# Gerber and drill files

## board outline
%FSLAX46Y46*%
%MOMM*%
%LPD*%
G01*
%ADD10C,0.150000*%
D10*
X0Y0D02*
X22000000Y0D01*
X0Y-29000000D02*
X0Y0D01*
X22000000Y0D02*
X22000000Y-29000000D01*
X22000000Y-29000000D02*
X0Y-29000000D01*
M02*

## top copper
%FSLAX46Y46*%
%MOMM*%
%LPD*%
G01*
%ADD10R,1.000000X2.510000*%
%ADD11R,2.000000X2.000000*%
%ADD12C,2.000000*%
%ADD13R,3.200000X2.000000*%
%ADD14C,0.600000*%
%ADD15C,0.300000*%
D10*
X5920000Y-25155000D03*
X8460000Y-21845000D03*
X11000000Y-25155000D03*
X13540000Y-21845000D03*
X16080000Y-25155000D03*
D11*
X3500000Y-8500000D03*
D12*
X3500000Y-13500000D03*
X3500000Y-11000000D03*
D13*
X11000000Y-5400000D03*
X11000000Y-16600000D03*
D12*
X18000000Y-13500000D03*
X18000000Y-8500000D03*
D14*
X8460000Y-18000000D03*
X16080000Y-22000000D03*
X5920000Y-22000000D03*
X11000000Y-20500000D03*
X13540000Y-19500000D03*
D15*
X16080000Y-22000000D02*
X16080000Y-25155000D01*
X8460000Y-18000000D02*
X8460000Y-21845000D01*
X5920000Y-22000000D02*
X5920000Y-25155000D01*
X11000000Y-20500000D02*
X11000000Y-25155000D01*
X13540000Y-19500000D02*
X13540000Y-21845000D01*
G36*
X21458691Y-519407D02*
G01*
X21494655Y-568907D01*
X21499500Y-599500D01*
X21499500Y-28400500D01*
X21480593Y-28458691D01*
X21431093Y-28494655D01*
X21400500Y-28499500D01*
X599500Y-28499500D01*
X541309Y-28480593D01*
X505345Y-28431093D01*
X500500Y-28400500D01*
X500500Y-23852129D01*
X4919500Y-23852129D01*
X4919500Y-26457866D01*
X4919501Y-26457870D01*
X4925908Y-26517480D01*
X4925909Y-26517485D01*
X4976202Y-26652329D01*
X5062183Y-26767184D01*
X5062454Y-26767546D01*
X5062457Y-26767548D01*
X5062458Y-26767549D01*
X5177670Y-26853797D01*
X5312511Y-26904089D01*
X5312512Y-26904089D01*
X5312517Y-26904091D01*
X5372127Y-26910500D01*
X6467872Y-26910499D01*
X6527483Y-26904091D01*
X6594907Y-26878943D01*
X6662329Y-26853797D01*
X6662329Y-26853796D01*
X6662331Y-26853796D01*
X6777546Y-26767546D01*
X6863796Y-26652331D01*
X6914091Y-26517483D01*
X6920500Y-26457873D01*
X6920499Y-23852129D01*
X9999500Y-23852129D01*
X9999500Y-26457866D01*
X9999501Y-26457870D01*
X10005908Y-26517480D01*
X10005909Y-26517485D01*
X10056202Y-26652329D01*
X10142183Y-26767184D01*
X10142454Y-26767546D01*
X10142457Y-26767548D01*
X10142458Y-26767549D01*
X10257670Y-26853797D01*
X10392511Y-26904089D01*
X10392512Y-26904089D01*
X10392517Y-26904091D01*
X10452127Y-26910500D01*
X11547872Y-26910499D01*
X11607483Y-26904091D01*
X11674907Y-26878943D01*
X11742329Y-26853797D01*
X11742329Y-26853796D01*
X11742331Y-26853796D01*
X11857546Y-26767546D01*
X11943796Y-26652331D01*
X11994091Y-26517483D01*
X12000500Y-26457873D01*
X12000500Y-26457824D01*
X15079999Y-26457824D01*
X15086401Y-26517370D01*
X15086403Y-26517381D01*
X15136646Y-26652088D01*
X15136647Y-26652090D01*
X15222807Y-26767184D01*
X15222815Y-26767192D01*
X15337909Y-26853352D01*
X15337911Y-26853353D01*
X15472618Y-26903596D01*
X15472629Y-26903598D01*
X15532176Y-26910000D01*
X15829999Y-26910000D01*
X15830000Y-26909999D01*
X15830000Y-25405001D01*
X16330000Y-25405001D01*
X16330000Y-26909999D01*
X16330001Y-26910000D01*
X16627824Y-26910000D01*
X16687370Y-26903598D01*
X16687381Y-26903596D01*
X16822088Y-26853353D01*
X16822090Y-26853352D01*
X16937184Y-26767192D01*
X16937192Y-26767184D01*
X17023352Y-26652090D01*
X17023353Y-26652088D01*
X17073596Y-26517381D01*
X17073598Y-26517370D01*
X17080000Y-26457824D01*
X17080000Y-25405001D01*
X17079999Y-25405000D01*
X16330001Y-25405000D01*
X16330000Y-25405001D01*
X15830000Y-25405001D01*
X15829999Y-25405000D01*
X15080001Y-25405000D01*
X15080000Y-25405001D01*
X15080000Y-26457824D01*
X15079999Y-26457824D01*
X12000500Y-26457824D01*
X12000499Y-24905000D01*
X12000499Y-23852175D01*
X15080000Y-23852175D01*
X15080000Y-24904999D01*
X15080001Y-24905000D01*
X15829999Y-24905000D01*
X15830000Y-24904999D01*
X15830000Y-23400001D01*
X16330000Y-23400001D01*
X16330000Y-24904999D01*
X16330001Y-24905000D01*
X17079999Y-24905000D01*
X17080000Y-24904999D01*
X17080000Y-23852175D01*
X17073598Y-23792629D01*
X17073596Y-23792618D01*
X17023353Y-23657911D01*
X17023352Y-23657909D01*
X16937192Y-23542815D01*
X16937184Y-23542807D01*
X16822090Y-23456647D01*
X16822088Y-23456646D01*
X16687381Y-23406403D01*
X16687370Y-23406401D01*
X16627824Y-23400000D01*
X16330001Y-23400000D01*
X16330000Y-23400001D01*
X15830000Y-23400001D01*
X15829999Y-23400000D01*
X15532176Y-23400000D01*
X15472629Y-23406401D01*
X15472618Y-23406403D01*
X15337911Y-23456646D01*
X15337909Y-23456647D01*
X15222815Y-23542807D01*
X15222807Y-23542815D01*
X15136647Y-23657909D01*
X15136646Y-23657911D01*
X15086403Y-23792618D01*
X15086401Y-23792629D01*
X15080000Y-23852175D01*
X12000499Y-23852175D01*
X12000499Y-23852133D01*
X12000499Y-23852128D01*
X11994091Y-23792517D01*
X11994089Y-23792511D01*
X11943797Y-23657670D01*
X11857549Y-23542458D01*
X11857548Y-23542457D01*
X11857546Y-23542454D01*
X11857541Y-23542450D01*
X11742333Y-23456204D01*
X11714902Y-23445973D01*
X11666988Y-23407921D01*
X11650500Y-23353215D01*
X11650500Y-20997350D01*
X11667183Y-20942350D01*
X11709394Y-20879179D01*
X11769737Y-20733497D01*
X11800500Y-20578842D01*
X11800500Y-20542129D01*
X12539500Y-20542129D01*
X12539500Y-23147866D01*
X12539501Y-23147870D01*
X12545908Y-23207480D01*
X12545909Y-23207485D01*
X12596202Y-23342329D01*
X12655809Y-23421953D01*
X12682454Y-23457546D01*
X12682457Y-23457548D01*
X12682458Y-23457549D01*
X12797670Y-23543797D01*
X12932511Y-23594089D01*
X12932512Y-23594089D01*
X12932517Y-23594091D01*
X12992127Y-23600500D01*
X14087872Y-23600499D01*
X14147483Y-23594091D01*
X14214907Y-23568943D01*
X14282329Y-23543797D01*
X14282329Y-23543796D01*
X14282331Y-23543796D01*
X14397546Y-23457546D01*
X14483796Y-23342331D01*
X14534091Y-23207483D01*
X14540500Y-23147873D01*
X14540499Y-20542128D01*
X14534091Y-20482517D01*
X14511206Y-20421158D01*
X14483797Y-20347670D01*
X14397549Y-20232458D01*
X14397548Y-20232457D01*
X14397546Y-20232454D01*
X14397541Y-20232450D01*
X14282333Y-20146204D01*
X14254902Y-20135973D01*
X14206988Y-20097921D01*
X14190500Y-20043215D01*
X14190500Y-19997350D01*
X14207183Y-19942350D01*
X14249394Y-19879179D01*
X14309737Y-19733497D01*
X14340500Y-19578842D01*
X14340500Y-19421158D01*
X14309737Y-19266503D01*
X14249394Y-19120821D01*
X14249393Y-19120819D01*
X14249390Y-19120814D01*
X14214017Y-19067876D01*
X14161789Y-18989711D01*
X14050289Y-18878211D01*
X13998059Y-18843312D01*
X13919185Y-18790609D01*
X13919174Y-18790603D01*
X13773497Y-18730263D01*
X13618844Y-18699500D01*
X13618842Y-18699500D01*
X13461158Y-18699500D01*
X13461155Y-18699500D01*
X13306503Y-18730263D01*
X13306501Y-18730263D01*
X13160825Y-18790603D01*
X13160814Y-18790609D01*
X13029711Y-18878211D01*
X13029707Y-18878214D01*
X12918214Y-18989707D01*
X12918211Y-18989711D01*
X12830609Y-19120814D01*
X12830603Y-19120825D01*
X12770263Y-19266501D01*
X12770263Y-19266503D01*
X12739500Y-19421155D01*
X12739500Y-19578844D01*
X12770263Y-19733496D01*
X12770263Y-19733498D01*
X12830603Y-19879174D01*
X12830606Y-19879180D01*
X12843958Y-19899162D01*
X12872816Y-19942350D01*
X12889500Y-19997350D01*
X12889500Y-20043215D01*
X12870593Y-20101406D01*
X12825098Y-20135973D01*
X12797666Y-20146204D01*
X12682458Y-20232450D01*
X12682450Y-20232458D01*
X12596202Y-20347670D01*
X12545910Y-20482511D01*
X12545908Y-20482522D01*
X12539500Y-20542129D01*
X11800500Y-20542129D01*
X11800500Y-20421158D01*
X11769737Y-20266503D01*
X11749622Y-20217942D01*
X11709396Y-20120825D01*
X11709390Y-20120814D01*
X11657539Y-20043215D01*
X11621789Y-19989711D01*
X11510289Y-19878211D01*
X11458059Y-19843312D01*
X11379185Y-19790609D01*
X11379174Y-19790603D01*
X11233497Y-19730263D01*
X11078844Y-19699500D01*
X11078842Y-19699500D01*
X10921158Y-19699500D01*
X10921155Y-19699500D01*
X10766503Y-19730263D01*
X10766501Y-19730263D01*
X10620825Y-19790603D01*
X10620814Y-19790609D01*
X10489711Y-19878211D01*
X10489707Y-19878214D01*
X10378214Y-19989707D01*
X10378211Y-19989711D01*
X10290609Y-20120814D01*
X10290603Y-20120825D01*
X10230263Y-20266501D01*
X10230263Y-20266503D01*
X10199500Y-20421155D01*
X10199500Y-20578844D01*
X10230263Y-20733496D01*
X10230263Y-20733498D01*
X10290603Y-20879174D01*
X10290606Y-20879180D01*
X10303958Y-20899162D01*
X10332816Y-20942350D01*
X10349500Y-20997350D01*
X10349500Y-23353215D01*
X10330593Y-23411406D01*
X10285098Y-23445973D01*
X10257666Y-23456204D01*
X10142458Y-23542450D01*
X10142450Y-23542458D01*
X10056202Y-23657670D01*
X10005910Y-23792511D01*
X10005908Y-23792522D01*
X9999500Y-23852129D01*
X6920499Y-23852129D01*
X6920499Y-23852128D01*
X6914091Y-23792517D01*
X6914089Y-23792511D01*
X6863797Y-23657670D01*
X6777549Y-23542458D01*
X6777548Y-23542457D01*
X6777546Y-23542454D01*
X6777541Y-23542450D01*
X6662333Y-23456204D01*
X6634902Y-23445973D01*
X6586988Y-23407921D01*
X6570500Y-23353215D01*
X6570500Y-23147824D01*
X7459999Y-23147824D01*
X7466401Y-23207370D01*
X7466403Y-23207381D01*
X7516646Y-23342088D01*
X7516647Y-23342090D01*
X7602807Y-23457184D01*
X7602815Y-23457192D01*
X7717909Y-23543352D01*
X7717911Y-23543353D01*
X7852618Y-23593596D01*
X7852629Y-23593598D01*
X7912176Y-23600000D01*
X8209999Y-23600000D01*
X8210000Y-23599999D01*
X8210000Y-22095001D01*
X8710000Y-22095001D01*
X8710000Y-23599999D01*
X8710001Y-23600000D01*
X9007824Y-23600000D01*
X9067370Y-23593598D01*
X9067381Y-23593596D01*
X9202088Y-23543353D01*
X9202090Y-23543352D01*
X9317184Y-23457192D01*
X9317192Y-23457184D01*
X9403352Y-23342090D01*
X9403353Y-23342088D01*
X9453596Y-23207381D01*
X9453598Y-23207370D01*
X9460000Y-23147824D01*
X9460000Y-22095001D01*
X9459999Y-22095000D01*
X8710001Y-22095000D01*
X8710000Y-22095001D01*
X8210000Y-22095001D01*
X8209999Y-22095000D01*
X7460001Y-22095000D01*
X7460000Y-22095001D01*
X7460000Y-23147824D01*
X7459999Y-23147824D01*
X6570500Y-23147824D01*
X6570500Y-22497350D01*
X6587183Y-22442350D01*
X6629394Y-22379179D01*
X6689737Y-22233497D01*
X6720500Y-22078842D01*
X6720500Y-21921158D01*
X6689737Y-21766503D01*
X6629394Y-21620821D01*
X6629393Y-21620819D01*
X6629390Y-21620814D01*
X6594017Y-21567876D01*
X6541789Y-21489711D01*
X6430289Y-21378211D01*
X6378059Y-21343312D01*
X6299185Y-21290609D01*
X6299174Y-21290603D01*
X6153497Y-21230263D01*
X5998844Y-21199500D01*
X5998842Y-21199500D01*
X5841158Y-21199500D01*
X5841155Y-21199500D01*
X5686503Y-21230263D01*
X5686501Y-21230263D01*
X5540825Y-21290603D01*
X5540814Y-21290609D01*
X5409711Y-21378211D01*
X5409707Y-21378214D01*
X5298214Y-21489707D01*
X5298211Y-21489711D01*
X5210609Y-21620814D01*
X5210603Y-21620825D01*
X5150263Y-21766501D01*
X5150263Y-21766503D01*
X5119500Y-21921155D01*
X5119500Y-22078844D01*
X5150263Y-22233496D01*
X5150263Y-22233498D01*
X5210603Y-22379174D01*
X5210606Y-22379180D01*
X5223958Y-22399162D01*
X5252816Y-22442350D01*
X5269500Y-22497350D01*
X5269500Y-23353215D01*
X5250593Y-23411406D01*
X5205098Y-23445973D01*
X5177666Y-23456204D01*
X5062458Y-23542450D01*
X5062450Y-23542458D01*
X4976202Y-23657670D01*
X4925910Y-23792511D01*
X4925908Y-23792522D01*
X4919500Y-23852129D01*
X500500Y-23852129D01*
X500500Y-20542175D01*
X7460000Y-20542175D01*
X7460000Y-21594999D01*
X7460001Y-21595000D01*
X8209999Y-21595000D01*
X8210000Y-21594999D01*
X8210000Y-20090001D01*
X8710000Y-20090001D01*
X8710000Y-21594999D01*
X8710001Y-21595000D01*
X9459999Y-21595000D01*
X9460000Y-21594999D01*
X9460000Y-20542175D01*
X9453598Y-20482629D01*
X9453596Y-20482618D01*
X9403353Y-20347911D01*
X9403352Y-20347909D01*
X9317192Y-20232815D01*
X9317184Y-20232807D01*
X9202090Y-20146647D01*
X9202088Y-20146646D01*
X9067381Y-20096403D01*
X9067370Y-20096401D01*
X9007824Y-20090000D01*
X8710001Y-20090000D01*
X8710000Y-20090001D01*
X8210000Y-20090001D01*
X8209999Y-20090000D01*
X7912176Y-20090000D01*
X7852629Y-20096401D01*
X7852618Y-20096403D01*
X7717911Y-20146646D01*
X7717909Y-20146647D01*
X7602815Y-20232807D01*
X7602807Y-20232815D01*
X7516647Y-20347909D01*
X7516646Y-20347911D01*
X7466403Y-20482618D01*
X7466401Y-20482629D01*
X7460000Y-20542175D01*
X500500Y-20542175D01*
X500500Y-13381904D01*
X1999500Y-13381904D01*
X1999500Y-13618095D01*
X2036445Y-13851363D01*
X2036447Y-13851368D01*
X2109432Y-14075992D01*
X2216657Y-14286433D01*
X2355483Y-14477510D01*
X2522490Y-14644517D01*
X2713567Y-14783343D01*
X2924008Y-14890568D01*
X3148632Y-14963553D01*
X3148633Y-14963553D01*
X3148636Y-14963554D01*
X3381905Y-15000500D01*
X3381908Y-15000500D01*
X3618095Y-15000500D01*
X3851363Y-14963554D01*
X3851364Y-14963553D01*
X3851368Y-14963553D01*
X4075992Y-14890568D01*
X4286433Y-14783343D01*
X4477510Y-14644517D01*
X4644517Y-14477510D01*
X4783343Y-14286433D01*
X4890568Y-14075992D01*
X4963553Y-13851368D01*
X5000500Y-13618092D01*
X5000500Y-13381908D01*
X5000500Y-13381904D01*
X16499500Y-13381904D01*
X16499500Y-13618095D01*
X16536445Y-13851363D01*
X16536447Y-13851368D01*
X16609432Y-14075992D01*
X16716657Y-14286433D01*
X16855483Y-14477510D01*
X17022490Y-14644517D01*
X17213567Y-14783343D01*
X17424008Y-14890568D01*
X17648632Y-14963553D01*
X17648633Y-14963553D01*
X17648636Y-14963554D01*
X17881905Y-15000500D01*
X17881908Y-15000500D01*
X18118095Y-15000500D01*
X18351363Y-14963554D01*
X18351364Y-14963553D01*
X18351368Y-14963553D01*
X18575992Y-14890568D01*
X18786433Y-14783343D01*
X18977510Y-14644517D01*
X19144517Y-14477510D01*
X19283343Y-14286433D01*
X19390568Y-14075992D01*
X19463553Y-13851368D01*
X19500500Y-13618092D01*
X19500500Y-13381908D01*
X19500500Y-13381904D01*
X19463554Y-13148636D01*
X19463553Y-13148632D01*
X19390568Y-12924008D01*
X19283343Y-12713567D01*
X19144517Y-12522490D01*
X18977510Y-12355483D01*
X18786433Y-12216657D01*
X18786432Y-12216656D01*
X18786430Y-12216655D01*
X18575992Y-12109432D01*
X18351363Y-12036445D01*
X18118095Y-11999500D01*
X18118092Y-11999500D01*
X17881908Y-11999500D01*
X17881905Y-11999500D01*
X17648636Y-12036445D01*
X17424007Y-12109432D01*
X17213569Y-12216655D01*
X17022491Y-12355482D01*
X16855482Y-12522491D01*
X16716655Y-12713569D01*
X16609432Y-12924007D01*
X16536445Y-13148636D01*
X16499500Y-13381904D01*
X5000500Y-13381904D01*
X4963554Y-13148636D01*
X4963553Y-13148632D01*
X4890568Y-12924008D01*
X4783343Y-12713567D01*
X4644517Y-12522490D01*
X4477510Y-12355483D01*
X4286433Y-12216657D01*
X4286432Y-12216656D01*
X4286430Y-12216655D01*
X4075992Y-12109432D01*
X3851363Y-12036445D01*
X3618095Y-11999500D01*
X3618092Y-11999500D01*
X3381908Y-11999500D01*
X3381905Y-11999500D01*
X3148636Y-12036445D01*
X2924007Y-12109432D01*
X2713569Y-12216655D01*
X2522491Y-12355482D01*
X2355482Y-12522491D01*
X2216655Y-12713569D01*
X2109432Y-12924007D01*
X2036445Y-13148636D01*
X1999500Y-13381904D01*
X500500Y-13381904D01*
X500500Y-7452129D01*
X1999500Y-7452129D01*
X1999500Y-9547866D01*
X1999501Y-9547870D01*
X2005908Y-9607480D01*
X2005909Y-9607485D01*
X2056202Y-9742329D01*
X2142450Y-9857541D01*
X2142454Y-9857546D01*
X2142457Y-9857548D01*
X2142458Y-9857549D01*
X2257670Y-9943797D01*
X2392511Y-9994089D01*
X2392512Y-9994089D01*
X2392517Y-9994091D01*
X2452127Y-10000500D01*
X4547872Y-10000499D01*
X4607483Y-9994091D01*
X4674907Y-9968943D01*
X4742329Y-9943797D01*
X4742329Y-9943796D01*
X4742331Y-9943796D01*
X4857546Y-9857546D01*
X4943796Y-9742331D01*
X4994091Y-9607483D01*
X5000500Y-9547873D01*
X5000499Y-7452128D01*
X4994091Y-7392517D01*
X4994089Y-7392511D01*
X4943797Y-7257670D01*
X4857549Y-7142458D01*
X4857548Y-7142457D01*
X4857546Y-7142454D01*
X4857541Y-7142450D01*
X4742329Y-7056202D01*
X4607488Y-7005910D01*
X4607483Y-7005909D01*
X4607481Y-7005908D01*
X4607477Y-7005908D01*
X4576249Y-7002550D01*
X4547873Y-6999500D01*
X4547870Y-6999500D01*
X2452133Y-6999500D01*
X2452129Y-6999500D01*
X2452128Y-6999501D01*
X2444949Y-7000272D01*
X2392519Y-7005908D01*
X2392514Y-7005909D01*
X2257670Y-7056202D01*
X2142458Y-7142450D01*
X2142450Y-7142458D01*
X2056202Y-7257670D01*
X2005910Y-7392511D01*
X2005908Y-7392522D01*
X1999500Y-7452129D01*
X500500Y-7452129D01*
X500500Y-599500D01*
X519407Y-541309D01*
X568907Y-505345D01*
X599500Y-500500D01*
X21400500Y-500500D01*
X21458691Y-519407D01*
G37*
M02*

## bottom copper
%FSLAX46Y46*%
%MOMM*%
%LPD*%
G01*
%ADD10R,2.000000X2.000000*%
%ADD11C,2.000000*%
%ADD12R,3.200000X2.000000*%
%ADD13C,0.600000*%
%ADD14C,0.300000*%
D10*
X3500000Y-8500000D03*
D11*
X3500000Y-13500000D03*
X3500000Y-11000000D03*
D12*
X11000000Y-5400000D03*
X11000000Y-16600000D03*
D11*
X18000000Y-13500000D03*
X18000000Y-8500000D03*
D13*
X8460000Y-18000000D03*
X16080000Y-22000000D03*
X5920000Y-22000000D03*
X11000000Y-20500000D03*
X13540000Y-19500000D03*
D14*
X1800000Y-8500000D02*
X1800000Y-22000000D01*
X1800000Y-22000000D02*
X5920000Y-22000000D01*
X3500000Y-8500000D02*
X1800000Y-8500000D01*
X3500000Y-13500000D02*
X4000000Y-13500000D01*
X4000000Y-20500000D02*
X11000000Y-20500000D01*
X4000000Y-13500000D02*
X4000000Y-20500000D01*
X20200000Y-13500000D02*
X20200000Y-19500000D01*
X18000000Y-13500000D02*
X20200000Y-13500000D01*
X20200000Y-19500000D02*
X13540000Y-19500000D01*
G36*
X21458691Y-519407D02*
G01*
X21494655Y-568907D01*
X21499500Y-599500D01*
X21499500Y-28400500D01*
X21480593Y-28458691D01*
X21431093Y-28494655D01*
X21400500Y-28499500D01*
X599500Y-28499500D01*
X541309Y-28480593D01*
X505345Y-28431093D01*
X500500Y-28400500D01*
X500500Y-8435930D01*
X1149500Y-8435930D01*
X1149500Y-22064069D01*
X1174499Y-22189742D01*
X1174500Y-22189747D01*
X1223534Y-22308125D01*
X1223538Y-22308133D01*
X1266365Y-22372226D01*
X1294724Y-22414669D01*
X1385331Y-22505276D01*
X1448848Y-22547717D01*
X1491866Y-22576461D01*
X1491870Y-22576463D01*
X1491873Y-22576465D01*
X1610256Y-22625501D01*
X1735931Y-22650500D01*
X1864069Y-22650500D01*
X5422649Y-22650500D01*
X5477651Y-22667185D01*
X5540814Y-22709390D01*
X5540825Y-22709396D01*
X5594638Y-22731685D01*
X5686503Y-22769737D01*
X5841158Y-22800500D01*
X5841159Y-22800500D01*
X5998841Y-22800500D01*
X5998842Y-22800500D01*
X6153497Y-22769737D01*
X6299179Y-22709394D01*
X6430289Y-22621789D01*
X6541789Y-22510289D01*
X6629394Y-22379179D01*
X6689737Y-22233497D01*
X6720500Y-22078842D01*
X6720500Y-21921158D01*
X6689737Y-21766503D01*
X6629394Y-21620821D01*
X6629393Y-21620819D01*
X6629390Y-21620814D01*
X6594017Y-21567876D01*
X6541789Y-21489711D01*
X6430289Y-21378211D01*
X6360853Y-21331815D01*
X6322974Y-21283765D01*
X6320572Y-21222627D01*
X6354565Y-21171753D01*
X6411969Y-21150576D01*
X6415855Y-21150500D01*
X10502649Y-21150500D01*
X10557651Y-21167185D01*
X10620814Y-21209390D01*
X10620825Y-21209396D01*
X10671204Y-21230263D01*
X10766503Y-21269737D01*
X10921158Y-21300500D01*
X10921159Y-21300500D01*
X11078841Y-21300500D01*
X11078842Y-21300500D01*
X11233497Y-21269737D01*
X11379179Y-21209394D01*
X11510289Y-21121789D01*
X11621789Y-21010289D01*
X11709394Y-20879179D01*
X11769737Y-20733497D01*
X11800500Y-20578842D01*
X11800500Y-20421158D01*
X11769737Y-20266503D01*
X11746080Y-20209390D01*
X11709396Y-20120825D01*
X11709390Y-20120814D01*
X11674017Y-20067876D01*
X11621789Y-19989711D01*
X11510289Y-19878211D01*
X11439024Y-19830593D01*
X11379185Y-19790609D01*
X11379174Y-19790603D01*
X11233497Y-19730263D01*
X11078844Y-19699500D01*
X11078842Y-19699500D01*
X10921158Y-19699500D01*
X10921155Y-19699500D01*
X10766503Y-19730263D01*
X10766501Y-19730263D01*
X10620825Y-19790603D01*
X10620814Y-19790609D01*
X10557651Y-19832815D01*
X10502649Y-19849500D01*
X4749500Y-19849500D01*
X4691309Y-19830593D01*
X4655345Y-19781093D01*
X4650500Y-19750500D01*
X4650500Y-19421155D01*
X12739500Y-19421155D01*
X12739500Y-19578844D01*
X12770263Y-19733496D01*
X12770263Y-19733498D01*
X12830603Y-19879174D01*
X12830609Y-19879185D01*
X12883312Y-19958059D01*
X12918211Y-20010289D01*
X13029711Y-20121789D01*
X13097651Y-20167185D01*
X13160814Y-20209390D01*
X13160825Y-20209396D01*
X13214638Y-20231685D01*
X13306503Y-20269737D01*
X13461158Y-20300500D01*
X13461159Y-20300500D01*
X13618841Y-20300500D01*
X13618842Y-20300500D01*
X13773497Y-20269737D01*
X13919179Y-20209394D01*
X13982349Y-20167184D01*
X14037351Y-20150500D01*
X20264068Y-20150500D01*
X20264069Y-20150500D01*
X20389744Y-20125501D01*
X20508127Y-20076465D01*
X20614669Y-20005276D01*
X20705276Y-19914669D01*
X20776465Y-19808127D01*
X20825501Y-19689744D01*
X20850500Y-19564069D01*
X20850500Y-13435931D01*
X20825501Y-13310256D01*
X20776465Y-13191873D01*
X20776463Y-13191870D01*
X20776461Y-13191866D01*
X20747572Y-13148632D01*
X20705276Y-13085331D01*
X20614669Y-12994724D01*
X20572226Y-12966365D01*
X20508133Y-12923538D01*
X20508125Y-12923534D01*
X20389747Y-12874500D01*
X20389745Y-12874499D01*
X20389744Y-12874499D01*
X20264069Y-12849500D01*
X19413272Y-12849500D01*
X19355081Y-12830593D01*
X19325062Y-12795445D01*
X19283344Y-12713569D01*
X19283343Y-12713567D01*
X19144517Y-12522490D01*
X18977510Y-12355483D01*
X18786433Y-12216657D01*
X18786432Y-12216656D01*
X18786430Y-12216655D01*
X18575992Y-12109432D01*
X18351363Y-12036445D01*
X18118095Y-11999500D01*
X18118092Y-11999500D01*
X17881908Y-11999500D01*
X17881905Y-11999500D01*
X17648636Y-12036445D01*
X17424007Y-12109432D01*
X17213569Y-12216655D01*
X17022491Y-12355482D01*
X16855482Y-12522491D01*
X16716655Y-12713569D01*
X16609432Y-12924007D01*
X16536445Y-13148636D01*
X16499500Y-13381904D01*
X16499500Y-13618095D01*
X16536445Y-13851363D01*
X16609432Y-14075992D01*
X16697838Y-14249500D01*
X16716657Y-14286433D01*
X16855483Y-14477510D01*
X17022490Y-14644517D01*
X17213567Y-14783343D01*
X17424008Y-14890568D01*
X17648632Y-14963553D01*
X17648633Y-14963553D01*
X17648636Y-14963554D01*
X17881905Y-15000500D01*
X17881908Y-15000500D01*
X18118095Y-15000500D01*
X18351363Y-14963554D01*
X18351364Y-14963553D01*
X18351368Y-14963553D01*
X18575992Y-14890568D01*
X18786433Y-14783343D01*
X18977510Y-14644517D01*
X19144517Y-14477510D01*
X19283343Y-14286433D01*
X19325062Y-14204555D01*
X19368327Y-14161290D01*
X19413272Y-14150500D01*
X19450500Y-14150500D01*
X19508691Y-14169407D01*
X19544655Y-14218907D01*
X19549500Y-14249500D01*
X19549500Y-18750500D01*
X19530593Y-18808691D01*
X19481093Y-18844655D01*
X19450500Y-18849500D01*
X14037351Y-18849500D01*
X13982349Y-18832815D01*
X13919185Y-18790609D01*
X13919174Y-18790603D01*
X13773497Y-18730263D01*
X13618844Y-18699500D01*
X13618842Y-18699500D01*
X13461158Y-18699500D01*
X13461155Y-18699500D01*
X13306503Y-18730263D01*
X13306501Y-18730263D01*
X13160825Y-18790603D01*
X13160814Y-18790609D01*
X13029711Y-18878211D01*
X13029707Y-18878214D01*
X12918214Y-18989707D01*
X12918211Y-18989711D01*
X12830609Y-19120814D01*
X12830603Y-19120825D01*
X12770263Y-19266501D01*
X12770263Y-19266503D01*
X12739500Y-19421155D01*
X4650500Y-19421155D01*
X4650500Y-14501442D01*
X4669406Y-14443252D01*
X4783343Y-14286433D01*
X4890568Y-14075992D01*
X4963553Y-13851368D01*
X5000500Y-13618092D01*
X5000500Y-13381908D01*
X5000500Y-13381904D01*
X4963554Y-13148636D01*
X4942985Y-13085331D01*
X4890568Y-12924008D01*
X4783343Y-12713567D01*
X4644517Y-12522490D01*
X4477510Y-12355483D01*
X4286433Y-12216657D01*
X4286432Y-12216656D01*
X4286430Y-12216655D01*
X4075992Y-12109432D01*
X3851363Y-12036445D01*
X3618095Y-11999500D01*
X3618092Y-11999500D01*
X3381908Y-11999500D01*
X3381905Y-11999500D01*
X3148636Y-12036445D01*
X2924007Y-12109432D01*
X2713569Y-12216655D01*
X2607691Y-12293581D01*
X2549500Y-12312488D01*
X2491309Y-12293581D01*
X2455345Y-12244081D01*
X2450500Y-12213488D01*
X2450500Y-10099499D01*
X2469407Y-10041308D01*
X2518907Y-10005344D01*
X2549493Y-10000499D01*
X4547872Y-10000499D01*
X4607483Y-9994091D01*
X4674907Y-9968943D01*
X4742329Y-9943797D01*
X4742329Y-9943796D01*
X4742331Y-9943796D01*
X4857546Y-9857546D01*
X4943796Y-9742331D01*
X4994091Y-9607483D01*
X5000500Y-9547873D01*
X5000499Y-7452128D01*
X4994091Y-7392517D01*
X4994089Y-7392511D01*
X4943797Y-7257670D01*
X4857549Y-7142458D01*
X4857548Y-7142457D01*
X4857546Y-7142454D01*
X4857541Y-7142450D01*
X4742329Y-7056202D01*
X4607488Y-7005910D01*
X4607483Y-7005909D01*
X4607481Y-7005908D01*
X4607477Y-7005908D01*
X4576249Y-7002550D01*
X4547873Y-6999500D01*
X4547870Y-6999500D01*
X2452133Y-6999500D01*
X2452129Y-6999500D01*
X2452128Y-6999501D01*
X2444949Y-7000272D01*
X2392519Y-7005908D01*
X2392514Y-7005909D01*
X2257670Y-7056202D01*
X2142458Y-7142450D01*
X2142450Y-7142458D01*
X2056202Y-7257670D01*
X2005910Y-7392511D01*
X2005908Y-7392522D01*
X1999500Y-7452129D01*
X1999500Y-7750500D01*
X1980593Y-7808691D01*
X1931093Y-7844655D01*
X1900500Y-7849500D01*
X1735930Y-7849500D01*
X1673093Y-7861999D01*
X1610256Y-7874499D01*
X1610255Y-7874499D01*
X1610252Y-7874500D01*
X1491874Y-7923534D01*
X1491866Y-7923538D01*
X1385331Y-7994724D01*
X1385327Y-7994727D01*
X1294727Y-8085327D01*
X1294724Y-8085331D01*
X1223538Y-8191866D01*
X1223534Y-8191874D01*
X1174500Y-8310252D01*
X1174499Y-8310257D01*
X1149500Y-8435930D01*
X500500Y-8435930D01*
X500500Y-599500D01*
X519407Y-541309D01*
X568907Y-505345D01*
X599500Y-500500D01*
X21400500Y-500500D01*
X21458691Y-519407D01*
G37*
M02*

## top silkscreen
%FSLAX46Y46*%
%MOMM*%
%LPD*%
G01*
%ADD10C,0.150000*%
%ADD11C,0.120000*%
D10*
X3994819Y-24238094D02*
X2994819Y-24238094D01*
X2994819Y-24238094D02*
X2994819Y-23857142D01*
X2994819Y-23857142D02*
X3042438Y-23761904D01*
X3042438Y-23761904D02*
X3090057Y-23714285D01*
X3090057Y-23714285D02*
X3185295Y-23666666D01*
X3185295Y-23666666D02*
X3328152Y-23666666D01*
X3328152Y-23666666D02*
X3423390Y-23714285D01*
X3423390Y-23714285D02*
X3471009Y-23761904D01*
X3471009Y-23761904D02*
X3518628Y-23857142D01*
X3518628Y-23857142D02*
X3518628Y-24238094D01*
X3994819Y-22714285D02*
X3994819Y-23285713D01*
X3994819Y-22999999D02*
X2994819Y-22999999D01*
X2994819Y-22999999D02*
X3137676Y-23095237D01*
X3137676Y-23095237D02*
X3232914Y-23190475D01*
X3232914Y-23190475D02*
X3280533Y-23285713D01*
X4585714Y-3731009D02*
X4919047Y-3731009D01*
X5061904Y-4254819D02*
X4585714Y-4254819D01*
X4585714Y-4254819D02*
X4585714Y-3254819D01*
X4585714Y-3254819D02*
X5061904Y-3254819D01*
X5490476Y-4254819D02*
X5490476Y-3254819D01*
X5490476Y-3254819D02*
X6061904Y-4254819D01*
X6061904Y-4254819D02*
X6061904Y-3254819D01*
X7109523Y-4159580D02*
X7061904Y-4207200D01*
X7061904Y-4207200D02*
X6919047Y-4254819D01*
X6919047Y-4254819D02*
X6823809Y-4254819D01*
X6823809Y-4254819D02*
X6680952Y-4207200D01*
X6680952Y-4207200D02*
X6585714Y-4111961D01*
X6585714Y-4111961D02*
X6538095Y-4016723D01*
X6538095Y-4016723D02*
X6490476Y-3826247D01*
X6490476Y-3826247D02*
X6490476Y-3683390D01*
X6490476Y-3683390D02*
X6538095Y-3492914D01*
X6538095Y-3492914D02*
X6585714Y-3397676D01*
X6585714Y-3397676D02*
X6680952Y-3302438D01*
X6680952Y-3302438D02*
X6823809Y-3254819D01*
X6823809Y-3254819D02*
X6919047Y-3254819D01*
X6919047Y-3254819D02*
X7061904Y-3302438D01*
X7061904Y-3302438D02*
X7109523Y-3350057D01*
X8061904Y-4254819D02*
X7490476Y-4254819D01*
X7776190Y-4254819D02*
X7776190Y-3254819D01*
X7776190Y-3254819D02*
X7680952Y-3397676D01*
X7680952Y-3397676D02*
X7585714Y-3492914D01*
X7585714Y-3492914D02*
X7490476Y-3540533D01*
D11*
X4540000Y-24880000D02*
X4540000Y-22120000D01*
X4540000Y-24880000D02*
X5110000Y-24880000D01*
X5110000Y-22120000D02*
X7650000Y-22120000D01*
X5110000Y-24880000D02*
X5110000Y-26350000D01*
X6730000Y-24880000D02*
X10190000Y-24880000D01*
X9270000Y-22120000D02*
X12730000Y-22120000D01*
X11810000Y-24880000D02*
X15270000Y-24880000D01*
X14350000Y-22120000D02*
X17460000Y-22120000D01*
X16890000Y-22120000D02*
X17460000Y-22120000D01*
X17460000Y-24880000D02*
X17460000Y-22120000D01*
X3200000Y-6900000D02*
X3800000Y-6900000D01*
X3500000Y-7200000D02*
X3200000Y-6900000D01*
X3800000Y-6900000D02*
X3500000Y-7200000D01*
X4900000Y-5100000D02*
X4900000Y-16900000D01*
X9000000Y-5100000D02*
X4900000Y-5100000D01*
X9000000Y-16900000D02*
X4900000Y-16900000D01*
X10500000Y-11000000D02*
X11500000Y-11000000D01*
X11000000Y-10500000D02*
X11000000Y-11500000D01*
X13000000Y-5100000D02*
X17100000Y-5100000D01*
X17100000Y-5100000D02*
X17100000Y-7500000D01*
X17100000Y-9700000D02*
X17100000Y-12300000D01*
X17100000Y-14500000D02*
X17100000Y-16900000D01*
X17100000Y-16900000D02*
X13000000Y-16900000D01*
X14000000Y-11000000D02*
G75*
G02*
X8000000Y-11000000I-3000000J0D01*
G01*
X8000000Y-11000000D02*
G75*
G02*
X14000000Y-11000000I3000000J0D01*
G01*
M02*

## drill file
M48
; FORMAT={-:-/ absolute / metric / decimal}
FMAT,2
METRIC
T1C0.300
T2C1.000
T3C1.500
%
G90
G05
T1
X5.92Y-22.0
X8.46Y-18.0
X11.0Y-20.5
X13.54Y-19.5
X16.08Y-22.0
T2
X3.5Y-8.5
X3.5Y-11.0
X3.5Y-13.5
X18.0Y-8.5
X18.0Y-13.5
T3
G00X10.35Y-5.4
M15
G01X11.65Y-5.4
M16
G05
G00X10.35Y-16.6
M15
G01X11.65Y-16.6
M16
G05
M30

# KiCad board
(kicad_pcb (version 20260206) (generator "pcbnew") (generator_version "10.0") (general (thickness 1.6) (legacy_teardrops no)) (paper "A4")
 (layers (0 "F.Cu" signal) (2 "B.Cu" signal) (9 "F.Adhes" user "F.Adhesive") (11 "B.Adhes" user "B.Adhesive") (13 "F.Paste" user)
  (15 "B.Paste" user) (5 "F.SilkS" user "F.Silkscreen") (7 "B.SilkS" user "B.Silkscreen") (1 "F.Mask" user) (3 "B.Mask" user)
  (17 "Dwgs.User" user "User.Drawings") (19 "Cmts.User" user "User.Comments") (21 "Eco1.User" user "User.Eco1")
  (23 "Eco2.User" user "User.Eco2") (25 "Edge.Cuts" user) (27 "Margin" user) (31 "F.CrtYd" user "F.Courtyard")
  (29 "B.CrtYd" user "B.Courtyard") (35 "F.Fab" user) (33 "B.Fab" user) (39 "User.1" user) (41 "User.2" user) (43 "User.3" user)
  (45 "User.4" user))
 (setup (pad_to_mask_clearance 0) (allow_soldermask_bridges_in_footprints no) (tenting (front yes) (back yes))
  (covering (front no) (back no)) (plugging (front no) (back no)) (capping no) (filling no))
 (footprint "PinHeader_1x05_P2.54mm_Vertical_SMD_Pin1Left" (layer "F.Cu") (at 11 23.5 90)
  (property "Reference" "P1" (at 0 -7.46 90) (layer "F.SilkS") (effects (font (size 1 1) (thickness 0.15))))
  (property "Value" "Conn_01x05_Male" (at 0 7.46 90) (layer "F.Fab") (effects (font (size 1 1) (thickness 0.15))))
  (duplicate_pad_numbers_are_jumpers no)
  (fp_line (start -1.38 -6.46) (end 1.38 -6.46) (stroke (width 0.12) (type solid)) (layer "F.SilkS"))
  (fp_line (start -1.38 -6.46) (end -1.38 -5.89) (stroke (width 0.12) (type solid)) (layer "F.SilkS"))
  (fp_line (start 1.38 -5.89) (end 1.38 -3.35) (stroke (width 0.12) (type solid)) (layer "F.SilkS"))
  (fp_line (start -1.38 -5.89) (end -2.85 -5.89) (stroke (width 0.12) (type solid)) (layer "F.SilkS"))
  (fp_line (start -1.38 -4.27) (end -1.38 -0.81) (stroke (width 0.12) (type solid)) (layer "F.SilkS"))
  (fp_line (start 1.38 -1.73) (end 1.38 1.73) (stroke (width 0.12) (type solid)) (layer "F.SilkS"))
  (fp_line (start -1.38 0.81) (end -1.38 4.27) (stroke (width 0.12) (type solid)) (layer "F.SilkS"))
  (fp_line (start 1.38 3.35) (end 1.38 6.46) (stroke (width 0.12) (type solid)) (layer "F.SilkS"))
  (fp_line (start 1.38 5.89) (end 1.38 6.46) (stroke (width 0.12) (type solid)) (layer "F.SilkS"))
  (fp_line (start -1.38 6.46) (end 1.38 6.46) (stroke (width 0.12) (type solid)) (layer "F.SilkS"))
  (pad "1" smd rect (at -1.655 -5.08 90) (size 2.51 1) (layers "F.Cu" "F.Mask" "F.Paste") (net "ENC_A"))
  (pad "2" smd rect (at 1.655 -2.54 90) (size 2.51 1) (layers "F.Cu" "F.Mask" "F.Paste") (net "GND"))
  (pad "3" smd rect (at -1.655 0 90) (size 2.51 1) (layers "F.Cu" "F.Mask" "F.Paste") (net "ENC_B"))
  (pad "4" smd rect (at 1.655 2.54 90) (size 2.51 1) (layers "F.Cu" "F.Mask" "F.Paste") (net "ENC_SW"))
  (pad "5" smd rect (at -1.655 5.08 90) (size 2.51 1) (layers "F.Cu" "F.Mask" "F.Paste") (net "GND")))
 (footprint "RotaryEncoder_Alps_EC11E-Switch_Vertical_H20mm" (layer "F.Cu") (at 3.5 8.5)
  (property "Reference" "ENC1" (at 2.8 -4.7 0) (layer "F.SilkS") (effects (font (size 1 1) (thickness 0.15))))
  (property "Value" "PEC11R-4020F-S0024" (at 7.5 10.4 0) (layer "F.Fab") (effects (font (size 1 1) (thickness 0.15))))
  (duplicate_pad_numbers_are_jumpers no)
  (fp_line (start -0.3 -1.6) (end 0.3 -1.6) (stroke (width 0.12) (type solid)) (layer "F.SilkS"))
  (fp_line (start 0 -1.3) (end -0.3 -1.6) (stroke (width 0.12) (type solid)) (layer "F.SilkS"))
  (fp_line (start 0.3 -1.6) (end 0 -1.3) (stroke (width 0.12) (type solid)) (layer "F.SilkS"))
  (fp_line (start 1.4 -3.4) (end 1.4 8.4) (stroke (width 0.12) (type solid)) (layer "F.SilkS"))
  (fp_line (start 5.5 -3.4) (end 1.4 -3.4) (stroke (width 0.12) (type solid)) (layer "F.SilkS"))
  (fp_line (start 5.5 8.4) (end 1.4 8.4) (stroke (width 0.12) (type solid)) (layer "F.SilkS"))
  (fp_line (start 7 2.5) (end 8 2.5) (stroke (width 0.12) (type solid)) (layer "F.SilkS"))
  (fp_line (start 7.5 2) (end 7.5 3) (stroke (width 0.12) (type solid)) (layer "F.SilkS"))
  (fp_line (start 9.5 -3.4) (end 13.6 -3.4) (stroke (width 0.12) (type solid)) (layer "F.SilkS"))
  (fp_line (start 13.6 -3.4) (end 13.6 -1) (stroke (width 0.12) (type solid)) (layer "F.SilkS"))
  (fp_line (start 13.6 1.2) (end 13.6 3.8) (stroke (width 0.12) (type solid)) (layer "F.SilkS"))
  (fp_line (start 13.6 6) (end 13.6 8.4) (stroke (width 0.12) (type solid)) (layer "F.SilkS"))
  (fp_line (start 13.6 8.4) (end 9.5 8.4) (stroke (width 0.12) (type solid)) (layer "F.SilkS"))
  (fp_circle (center 7.5 2.5) (end 10.5 2.5) (stroke (width 0.12) (type solid)) (fill no) (layer "F.SilkS"))
  (pad "A" thru_hole rect (at 0 0) (size 2 2) (drill 1) (layers "*.Cu" "*.Mask") (remove_unused_layers no) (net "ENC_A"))
  (pad "B" thru_hole circle (at 0 5) (size 2 2) (drill 1) (layers "*.Cu" "*.Mask") (remove_unused_layers no) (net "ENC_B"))
  (pad "C" thru_hole circle (at 0 2.5) (size 2 2) (drill 1) (layers "*.Cu" "*.Mask") (remove_unused_layers no) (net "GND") (zone_connect 2))
  (pad "MP" thru_hole rect (at 7.5 -3.1) (size 3.2 2) (drill oval 2.8 1.5) (layers "*.Cu" "*.Mask") (remove_unused_layers no) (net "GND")
   (zone_connect 2))
  (pad "MP" thru_hole rect (at 7.5 8.1) (size 3.2 2) (drill oval 2.8 1.5) (layers "*.Cu" "*.Mask") (remove_unused_layers no) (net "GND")
   (zone_connect 2))
  (pad "S1" thru_hole circle (at 14.5 5) (size 2 2) (drill 1) (layers "*.Cu" "*.Mask") (remove_unused_layers no) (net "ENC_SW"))
  (pad "S2" thru_hole circle (at 14.5 0) (size 2 2) (drill 1) (layers "*.Cu" "*.Mask") (remove_unused_layers no) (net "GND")
   (zone_connect 2)))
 (gr_line (start 0 0) (end 22 0) (stroke (width 0.15) (type default)) (layer "Edge.Cuts"))
 (gr_line (start 0 29) (end 0 0) (stroke (width 0.15) (type default)) (layer "Edge.Cuts"))
 (gr_line (start 22 0) (end 22 29) (stroke (width 0.15) (type default)) (layer "Edge.Cuts"))
 (gr_line (start 22 29) (end 0 29) (stroke (width 0.15) (type default)) (layer "Edge.Cuts"))
 (segment (start 5.92 22) (end 5.92 25.155) (width 0.3) (layer "F.Cu") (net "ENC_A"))
 (via (at 5.92 22) (size 0.6) (drill 0.3) (layers "F.Cu" "B.Cu") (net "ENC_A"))
 (segment (start 1.8 8.5) (end 1.8 22) (width 0.3) (layer "B.Cu") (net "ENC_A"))
 (segment (start 1.8 22) (end 5.92 22) (width 0.3) (layer "B.Cu") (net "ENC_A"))
 (segment (start 3.5 8.5) (end 1.8 8.5) (width 0.3) (layer "B.Cu") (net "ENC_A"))
 (segment (start 16.08 22) (end 16.08 25.155) (width 0.3) (layer "F.Cu") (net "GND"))
 (segment (start 8.46 18) (end 8.46 21.845) (width 0.3) (layer "F.Cu") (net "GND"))
 (via (at 8.46 18) (size 0.6) (drill 0.3) (layers "F.Cu" "B.Cu") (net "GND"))
 (via (at 16.08 22) (size 0.6) (drill 0.3) (layers "F.Cu" "B.Cu") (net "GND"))
 (segment (start 11 20.5) (end 11 25.155) (width 0.3) (layer "F.Cu") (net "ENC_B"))
 (via (at 11 20.5) (size 0.6) (drill 0.3) (layers "F.Cu" "B.Cu") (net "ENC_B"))
 (segment (start 3.5 13.5) (end 4 13.5) (width 0.3) (layer "B.Cu") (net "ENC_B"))
 (segment (start 4 20.5) (end 11 20.5) (width 0.3) (layer "B.Cu") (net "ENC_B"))
 (segment (start 4 13.5) (end 4 20.5) (width 0.3) (layer "B.Cu") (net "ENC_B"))
 (segment (start 13.54 19.5) (end 13.54 21.845) (width 0.3) (layer "F.Cu") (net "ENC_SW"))
 (via (at 13.54 19.5) (size 0.6) (drill 0.3) (layers "F.Cu" "B.Cu") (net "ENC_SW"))
 (segment (start 20.2 13.5) (end 20.2 19.5) (width 0.3) (layer "B.Cu") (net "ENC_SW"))
 (segment (start 18 13.5) (end 20.2 13.5) (width 0.3) (layer "B.Cu") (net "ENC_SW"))
 (segment (start 20.2 19.5) (end 13.54 19.5) (width 0.3) (layer "B.Cu") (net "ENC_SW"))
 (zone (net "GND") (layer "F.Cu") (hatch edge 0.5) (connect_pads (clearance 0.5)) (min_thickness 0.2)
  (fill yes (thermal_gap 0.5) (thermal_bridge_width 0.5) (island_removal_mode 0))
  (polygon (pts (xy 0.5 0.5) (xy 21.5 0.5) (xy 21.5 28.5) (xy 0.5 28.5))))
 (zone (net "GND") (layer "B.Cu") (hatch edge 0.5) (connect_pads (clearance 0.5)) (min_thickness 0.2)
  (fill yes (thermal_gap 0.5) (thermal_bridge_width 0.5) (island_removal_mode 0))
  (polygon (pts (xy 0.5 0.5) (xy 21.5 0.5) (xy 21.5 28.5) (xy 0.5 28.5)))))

